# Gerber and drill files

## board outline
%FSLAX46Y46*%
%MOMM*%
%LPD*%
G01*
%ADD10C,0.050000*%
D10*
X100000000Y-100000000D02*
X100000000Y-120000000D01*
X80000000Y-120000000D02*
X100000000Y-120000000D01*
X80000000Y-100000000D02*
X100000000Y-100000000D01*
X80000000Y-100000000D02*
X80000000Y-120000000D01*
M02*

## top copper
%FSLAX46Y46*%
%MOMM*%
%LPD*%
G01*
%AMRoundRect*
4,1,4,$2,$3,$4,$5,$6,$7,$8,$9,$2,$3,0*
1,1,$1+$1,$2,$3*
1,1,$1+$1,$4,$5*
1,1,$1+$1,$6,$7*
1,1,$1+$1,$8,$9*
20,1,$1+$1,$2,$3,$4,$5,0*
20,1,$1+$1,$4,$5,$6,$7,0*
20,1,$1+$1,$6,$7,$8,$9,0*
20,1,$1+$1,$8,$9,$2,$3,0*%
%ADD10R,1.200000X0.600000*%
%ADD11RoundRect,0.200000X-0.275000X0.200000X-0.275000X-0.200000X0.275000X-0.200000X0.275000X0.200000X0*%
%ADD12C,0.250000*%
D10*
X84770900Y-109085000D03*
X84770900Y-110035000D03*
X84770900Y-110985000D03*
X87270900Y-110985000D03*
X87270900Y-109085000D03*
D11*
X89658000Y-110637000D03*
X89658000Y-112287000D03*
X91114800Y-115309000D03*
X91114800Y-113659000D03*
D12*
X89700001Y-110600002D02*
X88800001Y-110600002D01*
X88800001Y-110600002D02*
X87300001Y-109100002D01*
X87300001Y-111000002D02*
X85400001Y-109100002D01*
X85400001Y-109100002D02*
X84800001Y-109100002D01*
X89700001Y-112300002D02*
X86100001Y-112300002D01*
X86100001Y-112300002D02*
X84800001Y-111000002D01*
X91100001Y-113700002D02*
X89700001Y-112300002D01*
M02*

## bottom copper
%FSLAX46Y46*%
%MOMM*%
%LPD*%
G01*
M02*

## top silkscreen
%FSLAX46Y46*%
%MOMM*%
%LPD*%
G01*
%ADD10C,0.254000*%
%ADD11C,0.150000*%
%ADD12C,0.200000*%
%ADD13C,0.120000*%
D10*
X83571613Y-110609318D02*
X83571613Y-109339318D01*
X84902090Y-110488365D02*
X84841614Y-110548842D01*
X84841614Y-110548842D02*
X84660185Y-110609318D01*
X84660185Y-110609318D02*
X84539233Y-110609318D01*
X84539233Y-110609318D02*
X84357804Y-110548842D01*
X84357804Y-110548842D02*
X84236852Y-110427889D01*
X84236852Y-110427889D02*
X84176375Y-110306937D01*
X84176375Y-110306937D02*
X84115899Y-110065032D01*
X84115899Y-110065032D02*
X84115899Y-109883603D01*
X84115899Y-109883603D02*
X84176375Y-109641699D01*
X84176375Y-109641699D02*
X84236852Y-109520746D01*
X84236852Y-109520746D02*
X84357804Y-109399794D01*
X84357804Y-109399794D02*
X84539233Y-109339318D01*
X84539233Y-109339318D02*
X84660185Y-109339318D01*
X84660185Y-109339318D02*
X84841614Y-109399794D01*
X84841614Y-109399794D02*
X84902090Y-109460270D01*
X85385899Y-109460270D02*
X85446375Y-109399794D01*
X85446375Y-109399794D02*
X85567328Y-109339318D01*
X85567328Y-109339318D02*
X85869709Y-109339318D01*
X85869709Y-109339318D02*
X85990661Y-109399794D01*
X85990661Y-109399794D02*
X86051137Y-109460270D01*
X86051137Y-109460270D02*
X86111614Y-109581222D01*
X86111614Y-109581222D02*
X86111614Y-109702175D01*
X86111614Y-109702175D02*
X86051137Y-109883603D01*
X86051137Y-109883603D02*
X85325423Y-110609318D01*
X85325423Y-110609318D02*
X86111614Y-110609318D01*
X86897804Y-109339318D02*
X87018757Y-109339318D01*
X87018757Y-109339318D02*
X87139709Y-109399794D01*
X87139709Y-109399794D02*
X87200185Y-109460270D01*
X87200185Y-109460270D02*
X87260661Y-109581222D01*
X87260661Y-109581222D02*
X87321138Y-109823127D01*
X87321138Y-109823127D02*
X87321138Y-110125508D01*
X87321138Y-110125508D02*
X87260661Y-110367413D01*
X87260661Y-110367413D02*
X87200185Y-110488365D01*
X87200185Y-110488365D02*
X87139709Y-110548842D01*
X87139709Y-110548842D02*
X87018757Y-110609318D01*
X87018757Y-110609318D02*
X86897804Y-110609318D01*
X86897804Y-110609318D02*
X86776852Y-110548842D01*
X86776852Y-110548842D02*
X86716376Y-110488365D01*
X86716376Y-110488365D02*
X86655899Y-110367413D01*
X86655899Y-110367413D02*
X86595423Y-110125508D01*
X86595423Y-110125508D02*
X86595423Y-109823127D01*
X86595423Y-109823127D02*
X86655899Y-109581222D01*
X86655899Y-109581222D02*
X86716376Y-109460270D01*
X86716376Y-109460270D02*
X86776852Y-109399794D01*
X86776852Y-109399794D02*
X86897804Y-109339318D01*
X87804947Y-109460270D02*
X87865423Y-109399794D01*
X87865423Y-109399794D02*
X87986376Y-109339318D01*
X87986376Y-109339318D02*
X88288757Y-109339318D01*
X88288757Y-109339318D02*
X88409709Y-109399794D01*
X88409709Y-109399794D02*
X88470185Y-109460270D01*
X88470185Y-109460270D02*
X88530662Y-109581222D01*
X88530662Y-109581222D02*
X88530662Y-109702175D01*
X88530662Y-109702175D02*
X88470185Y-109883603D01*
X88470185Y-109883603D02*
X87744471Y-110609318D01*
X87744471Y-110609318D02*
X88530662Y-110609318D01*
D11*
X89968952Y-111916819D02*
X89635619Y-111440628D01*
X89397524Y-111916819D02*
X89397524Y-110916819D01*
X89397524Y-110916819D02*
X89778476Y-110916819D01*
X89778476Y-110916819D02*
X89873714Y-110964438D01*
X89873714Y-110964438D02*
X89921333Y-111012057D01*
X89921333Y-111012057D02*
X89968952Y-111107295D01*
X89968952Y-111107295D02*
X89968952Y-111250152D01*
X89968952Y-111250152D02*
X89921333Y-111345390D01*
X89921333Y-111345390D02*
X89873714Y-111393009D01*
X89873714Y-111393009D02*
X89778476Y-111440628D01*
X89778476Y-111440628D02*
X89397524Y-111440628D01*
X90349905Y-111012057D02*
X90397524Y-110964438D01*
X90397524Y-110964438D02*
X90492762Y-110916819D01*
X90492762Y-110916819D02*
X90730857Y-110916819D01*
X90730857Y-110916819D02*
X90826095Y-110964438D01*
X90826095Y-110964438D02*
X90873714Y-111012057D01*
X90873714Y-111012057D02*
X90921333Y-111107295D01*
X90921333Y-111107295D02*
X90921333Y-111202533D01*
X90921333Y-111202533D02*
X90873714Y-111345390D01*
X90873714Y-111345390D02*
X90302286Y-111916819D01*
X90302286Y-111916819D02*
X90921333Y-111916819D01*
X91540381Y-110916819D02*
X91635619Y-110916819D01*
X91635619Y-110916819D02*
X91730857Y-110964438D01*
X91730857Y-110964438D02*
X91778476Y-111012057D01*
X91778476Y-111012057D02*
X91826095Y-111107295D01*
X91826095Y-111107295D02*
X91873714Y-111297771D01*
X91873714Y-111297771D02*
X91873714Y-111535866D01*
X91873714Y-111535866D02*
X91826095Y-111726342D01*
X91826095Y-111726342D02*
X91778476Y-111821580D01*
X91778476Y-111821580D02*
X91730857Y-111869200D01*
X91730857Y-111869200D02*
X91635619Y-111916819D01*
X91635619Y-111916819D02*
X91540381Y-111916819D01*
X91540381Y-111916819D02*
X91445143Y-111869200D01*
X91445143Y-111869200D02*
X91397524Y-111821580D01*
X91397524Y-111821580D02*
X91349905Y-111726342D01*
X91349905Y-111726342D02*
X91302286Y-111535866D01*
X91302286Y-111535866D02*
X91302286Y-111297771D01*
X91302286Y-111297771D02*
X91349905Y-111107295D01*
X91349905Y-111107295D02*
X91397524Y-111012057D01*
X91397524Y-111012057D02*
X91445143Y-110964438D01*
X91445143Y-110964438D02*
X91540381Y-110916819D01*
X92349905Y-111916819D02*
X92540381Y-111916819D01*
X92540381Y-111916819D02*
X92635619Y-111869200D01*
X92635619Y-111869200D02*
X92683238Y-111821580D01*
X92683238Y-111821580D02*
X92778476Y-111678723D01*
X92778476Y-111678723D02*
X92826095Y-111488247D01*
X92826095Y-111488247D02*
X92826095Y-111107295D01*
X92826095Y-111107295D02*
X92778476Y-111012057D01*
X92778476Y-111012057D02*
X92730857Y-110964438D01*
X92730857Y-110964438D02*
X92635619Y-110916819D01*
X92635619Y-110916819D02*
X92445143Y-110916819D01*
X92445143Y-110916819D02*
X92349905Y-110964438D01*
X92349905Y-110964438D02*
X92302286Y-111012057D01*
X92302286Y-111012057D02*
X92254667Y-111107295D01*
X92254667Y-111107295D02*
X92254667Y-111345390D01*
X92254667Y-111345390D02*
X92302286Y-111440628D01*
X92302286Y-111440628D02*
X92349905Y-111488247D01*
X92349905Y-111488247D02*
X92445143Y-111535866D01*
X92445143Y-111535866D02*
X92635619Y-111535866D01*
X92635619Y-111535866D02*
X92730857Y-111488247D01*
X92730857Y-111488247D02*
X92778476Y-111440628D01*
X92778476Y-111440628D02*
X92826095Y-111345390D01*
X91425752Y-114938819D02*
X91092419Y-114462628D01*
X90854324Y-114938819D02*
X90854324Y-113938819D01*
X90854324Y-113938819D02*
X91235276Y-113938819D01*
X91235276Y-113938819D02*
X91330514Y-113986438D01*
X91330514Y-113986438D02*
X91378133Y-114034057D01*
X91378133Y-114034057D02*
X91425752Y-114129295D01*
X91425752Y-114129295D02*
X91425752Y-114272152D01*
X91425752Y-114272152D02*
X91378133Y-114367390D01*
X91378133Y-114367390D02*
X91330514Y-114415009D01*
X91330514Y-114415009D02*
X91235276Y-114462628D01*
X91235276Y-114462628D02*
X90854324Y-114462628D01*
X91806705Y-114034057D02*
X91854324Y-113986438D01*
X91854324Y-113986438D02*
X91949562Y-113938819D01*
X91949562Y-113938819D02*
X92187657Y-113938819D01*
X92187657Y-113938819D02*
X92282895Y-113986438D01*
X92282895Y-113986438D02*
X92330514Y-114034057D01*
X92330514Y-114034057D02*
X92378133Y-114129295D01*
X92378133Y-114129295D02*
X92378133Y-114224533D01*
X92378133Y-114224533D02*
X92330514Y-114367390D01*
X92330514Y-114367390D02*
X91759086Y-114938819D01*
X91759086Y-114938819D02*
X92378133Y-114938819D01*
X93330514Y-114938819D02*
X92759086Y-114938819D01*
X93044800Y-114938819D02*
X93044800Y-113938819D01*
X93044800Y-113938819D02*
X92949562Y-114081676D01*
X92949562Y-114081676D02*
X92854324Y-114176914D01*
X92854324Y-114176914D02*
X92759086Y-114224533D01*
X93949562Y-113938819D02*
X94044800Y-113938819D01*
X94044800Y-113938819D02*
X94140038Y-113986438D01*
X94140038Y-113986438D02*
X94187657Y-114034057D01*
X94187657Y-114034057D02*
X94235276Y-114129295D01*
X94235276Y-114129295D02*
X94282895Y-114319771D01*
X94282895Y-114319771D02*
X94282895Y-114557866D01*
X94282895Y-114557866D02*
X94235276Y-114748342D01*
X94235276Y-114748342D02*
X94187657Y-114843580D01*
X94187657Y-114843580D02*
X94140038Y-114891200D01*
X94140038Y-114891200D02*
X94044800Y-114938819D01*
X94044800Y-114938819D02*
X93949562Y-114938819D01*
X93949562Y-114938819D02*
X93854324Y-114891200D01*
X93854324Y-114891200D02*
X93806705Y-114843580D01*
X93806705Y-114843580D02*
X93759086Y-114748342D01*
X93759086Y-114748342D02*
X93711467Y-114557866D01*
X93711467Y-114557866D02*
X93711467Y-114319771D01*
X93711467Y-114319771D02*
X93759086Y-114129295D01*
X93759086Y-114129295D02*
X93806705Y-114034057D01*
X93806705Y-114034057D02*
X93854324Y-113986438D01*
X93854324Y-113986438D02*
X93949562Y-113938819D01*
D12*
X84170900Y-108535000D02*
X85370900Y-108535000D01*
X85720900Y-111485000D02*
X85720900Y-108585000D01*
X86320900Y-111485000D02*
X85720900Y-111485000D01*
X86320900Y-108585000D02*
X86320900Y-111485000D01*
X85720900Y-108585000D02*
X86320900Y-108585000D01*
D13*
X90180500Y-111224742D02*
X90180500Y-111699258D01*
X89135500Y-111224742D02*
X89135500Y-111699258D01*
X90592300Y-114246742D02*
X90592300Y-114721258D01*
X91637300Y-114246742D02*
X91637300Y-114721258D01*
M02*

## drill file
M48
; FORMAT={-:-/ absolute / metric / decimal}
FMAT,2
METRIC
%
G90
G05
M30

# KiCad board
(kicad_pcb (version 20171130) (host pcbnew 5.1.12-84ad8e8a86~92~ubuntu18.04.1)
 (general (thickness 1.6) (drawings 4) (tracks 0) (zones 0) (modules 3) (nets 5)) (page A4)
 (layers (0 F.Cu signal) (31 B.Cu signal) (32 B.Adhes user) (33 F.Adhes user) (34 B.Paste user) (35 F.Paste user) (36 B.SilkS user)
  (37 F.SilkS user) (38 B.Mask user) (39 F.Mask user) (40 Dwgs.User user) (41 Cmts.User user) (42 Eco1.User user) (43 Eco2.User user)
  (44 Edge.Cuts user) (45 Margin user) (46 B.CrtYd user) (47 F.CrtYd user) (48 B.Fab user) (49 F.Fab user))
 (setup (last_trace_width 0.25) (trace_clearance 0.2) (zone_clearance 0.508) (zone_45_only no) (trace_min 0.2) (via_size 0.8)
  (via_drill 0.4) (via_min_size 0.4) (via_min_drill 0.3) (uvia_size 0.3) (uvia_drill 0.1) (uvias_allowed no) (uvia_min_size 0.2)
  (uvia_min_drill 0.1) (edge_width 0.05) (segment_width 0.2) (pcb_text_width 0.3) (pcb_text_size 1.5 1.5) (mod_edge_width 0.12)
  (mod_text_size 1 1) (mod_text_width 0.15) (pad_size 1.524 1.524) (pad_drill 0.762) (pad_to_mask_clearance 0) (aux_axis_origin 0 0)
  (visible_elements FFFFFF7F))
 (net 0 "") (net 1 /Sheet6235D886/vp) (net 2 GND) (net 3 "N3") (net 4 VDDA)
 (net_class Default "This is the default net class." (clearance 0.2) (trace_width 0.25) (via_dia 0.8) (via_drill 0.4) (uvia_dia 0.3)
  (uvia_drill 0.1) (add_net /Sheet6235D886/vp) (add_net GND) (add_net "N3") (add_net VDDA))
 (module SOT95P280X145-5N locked (layer F.Cu) (at 86.020900 110.035000)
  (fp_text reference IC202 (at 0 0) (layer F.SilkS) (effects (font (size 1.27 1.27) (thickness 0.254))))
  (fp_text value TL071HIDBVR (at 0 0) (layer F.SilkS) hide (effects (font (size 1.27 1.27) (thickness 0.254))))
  (fp_line (start -1.85 -1.5) (end -0.65 -1.5) (layer F.SilkS) (width 0.2))
  (fp_line (start -0.3 1.45) (end -0.3 -1.45) (layer F.SilkS) (width 0.2))
  (fp_line (start 0.3 1.45) (end -0.3 1.45) (layer F.SilkS) (width 0.2))
  (fp_line (start 0.3 -1.45) (end 0.3 1.45) (layer F.SilkS) (width 0.2))
  (fp_line (start -0.3 -1.45) (end 0.3 -1.45) (layer F.SilkS) (width 0.2))
  (pad 1 smd rect (at -1.25 -0.95 90.000000) (size 0.6 1.2) (layers F.Cu F.Mask F.Paste) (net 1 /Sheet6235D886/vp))
  (pad 2 smd rect (at -1.25 0 90.000000) (size 0.6 1.2) (layers F.Cu F.Mask F.Paste) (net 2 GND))
  (pad 3 smd rect (at -1.25 0.95 90.000000) (size 0.6 1.2) (layers F.Cu F.Mask F.Paste) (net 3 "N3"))
  (pad 4 smd rect (at 1.25 0.95 90.000000) (size 0.6 1.2) (layers F.Cu F.Mask F.Paste) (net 1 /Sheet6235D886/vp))
  (pad 5 smd rect (at 1.25 -0.95 90.000000) (size 0.6 1.2) (layers F.Cu F.Mask F.Paste) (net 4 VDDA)))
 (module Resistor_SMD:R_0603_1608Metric (layer F.Cu) (at 89.658000 111.462000 270.000000)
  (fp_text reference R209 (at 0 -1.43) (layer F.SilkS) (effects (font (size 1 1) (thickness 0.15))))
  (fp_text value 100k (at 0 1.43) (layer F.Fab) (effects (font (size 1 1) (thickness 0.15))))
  (fp_line (start -0.237258 -0.5225) (end 0.237258 -0.5225) (layer F.SilkS) (width 0.12))
  (fp_line (start -0.237258 0.5225) (end 0.237258 0.5225) (layer F.SilkS) (width 0.12))
  (pad 1 smd roundrect (at -0.825 0 270.000000) (size 0.8 0.95) (layers F.Cu F.Mask F.Paste) (roundrect_rratio 0.25) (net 4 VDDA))
  (pad 2 smd roundrect (at 0.825 0 270.000000) (size 0.8 0.95) (layers F.Cu F.Mask F.Paste) (roundrect_rratio 0.25) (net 3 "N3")))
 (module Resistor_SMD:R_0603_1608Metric (layer F.Cu) (at 91.114800 114.484000 270.000000)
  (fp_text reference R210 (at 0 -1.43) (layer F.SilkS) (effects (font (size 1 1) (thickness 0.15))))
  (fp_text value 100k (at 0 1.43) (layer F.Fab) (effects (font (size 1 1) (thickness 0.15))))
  (fp_line (start -0.237258 0.5225) (end 0.237258 0.5225) (layer F.SilkS) (width 0.12))
  (fp_line (start -0.237258 -0.5225) (end 0.237258 -0.5225) (layer F.SilkS) (width 0.12))
  (pad 2 smd roundrect (at 0.825 0 270.000000) (size 0.8 0.95) (layers F.Cu F.Mask F.Paste) (roundrect_rratio 0.25) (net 2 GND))
  (pad 1 smd roundrect (at -0.825 0 270.000000) (size 0.8 0.95) (layers F.Cu F.Mask F.Paste) (roundrect_rratio 0.25) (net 3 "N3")))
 (gr_line (start 100 100) (end 100 120) (layer Edge.Cuts) (width 0.05))
 (gr_line (start 80 120) (end 100 120) (layer Edge.Cuts) (width 0.05))
 (gr_line (start 80 100) (end 100 100) (layer Edge.Cuts) (width 0.05))
 (gr_line (start 80 100) (end 80 120) (layer Edge.Cuts) (width 0.05))
 (segment (start 89.700001 110.600002) (end 88.800001 110.600002) (width 0.250000) (layer F.Cu) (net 4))
 (segment (start 88.800001 110.600002) (end 87.300001 109.100002) (width 0.250000) (layer F.Cu) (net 4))
 (segment (start 87.300001 111.000002) (end 85.400001 109.100002) (width 0.250000) (layer F.Cu) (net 1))
 (segment (start 85.400001 109.100002) (end 84.800001 109.100002) (width 0.250000) (layer F.Cu) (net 1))
 (segment (start 89.700001 112.300002) (end 86.100001 112.300002) (width 0.250000) (layer F.Cu) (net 3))
 (segment (start 86.100001 112.300002) (end 84.800001 111.000002) (width 0.250000) (layer F.Cu) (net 3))
 (segment (start 91.100001 113.700002) (end 89.700001 112.300002) (width 0.250000) (layer F.Cu) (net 3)))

